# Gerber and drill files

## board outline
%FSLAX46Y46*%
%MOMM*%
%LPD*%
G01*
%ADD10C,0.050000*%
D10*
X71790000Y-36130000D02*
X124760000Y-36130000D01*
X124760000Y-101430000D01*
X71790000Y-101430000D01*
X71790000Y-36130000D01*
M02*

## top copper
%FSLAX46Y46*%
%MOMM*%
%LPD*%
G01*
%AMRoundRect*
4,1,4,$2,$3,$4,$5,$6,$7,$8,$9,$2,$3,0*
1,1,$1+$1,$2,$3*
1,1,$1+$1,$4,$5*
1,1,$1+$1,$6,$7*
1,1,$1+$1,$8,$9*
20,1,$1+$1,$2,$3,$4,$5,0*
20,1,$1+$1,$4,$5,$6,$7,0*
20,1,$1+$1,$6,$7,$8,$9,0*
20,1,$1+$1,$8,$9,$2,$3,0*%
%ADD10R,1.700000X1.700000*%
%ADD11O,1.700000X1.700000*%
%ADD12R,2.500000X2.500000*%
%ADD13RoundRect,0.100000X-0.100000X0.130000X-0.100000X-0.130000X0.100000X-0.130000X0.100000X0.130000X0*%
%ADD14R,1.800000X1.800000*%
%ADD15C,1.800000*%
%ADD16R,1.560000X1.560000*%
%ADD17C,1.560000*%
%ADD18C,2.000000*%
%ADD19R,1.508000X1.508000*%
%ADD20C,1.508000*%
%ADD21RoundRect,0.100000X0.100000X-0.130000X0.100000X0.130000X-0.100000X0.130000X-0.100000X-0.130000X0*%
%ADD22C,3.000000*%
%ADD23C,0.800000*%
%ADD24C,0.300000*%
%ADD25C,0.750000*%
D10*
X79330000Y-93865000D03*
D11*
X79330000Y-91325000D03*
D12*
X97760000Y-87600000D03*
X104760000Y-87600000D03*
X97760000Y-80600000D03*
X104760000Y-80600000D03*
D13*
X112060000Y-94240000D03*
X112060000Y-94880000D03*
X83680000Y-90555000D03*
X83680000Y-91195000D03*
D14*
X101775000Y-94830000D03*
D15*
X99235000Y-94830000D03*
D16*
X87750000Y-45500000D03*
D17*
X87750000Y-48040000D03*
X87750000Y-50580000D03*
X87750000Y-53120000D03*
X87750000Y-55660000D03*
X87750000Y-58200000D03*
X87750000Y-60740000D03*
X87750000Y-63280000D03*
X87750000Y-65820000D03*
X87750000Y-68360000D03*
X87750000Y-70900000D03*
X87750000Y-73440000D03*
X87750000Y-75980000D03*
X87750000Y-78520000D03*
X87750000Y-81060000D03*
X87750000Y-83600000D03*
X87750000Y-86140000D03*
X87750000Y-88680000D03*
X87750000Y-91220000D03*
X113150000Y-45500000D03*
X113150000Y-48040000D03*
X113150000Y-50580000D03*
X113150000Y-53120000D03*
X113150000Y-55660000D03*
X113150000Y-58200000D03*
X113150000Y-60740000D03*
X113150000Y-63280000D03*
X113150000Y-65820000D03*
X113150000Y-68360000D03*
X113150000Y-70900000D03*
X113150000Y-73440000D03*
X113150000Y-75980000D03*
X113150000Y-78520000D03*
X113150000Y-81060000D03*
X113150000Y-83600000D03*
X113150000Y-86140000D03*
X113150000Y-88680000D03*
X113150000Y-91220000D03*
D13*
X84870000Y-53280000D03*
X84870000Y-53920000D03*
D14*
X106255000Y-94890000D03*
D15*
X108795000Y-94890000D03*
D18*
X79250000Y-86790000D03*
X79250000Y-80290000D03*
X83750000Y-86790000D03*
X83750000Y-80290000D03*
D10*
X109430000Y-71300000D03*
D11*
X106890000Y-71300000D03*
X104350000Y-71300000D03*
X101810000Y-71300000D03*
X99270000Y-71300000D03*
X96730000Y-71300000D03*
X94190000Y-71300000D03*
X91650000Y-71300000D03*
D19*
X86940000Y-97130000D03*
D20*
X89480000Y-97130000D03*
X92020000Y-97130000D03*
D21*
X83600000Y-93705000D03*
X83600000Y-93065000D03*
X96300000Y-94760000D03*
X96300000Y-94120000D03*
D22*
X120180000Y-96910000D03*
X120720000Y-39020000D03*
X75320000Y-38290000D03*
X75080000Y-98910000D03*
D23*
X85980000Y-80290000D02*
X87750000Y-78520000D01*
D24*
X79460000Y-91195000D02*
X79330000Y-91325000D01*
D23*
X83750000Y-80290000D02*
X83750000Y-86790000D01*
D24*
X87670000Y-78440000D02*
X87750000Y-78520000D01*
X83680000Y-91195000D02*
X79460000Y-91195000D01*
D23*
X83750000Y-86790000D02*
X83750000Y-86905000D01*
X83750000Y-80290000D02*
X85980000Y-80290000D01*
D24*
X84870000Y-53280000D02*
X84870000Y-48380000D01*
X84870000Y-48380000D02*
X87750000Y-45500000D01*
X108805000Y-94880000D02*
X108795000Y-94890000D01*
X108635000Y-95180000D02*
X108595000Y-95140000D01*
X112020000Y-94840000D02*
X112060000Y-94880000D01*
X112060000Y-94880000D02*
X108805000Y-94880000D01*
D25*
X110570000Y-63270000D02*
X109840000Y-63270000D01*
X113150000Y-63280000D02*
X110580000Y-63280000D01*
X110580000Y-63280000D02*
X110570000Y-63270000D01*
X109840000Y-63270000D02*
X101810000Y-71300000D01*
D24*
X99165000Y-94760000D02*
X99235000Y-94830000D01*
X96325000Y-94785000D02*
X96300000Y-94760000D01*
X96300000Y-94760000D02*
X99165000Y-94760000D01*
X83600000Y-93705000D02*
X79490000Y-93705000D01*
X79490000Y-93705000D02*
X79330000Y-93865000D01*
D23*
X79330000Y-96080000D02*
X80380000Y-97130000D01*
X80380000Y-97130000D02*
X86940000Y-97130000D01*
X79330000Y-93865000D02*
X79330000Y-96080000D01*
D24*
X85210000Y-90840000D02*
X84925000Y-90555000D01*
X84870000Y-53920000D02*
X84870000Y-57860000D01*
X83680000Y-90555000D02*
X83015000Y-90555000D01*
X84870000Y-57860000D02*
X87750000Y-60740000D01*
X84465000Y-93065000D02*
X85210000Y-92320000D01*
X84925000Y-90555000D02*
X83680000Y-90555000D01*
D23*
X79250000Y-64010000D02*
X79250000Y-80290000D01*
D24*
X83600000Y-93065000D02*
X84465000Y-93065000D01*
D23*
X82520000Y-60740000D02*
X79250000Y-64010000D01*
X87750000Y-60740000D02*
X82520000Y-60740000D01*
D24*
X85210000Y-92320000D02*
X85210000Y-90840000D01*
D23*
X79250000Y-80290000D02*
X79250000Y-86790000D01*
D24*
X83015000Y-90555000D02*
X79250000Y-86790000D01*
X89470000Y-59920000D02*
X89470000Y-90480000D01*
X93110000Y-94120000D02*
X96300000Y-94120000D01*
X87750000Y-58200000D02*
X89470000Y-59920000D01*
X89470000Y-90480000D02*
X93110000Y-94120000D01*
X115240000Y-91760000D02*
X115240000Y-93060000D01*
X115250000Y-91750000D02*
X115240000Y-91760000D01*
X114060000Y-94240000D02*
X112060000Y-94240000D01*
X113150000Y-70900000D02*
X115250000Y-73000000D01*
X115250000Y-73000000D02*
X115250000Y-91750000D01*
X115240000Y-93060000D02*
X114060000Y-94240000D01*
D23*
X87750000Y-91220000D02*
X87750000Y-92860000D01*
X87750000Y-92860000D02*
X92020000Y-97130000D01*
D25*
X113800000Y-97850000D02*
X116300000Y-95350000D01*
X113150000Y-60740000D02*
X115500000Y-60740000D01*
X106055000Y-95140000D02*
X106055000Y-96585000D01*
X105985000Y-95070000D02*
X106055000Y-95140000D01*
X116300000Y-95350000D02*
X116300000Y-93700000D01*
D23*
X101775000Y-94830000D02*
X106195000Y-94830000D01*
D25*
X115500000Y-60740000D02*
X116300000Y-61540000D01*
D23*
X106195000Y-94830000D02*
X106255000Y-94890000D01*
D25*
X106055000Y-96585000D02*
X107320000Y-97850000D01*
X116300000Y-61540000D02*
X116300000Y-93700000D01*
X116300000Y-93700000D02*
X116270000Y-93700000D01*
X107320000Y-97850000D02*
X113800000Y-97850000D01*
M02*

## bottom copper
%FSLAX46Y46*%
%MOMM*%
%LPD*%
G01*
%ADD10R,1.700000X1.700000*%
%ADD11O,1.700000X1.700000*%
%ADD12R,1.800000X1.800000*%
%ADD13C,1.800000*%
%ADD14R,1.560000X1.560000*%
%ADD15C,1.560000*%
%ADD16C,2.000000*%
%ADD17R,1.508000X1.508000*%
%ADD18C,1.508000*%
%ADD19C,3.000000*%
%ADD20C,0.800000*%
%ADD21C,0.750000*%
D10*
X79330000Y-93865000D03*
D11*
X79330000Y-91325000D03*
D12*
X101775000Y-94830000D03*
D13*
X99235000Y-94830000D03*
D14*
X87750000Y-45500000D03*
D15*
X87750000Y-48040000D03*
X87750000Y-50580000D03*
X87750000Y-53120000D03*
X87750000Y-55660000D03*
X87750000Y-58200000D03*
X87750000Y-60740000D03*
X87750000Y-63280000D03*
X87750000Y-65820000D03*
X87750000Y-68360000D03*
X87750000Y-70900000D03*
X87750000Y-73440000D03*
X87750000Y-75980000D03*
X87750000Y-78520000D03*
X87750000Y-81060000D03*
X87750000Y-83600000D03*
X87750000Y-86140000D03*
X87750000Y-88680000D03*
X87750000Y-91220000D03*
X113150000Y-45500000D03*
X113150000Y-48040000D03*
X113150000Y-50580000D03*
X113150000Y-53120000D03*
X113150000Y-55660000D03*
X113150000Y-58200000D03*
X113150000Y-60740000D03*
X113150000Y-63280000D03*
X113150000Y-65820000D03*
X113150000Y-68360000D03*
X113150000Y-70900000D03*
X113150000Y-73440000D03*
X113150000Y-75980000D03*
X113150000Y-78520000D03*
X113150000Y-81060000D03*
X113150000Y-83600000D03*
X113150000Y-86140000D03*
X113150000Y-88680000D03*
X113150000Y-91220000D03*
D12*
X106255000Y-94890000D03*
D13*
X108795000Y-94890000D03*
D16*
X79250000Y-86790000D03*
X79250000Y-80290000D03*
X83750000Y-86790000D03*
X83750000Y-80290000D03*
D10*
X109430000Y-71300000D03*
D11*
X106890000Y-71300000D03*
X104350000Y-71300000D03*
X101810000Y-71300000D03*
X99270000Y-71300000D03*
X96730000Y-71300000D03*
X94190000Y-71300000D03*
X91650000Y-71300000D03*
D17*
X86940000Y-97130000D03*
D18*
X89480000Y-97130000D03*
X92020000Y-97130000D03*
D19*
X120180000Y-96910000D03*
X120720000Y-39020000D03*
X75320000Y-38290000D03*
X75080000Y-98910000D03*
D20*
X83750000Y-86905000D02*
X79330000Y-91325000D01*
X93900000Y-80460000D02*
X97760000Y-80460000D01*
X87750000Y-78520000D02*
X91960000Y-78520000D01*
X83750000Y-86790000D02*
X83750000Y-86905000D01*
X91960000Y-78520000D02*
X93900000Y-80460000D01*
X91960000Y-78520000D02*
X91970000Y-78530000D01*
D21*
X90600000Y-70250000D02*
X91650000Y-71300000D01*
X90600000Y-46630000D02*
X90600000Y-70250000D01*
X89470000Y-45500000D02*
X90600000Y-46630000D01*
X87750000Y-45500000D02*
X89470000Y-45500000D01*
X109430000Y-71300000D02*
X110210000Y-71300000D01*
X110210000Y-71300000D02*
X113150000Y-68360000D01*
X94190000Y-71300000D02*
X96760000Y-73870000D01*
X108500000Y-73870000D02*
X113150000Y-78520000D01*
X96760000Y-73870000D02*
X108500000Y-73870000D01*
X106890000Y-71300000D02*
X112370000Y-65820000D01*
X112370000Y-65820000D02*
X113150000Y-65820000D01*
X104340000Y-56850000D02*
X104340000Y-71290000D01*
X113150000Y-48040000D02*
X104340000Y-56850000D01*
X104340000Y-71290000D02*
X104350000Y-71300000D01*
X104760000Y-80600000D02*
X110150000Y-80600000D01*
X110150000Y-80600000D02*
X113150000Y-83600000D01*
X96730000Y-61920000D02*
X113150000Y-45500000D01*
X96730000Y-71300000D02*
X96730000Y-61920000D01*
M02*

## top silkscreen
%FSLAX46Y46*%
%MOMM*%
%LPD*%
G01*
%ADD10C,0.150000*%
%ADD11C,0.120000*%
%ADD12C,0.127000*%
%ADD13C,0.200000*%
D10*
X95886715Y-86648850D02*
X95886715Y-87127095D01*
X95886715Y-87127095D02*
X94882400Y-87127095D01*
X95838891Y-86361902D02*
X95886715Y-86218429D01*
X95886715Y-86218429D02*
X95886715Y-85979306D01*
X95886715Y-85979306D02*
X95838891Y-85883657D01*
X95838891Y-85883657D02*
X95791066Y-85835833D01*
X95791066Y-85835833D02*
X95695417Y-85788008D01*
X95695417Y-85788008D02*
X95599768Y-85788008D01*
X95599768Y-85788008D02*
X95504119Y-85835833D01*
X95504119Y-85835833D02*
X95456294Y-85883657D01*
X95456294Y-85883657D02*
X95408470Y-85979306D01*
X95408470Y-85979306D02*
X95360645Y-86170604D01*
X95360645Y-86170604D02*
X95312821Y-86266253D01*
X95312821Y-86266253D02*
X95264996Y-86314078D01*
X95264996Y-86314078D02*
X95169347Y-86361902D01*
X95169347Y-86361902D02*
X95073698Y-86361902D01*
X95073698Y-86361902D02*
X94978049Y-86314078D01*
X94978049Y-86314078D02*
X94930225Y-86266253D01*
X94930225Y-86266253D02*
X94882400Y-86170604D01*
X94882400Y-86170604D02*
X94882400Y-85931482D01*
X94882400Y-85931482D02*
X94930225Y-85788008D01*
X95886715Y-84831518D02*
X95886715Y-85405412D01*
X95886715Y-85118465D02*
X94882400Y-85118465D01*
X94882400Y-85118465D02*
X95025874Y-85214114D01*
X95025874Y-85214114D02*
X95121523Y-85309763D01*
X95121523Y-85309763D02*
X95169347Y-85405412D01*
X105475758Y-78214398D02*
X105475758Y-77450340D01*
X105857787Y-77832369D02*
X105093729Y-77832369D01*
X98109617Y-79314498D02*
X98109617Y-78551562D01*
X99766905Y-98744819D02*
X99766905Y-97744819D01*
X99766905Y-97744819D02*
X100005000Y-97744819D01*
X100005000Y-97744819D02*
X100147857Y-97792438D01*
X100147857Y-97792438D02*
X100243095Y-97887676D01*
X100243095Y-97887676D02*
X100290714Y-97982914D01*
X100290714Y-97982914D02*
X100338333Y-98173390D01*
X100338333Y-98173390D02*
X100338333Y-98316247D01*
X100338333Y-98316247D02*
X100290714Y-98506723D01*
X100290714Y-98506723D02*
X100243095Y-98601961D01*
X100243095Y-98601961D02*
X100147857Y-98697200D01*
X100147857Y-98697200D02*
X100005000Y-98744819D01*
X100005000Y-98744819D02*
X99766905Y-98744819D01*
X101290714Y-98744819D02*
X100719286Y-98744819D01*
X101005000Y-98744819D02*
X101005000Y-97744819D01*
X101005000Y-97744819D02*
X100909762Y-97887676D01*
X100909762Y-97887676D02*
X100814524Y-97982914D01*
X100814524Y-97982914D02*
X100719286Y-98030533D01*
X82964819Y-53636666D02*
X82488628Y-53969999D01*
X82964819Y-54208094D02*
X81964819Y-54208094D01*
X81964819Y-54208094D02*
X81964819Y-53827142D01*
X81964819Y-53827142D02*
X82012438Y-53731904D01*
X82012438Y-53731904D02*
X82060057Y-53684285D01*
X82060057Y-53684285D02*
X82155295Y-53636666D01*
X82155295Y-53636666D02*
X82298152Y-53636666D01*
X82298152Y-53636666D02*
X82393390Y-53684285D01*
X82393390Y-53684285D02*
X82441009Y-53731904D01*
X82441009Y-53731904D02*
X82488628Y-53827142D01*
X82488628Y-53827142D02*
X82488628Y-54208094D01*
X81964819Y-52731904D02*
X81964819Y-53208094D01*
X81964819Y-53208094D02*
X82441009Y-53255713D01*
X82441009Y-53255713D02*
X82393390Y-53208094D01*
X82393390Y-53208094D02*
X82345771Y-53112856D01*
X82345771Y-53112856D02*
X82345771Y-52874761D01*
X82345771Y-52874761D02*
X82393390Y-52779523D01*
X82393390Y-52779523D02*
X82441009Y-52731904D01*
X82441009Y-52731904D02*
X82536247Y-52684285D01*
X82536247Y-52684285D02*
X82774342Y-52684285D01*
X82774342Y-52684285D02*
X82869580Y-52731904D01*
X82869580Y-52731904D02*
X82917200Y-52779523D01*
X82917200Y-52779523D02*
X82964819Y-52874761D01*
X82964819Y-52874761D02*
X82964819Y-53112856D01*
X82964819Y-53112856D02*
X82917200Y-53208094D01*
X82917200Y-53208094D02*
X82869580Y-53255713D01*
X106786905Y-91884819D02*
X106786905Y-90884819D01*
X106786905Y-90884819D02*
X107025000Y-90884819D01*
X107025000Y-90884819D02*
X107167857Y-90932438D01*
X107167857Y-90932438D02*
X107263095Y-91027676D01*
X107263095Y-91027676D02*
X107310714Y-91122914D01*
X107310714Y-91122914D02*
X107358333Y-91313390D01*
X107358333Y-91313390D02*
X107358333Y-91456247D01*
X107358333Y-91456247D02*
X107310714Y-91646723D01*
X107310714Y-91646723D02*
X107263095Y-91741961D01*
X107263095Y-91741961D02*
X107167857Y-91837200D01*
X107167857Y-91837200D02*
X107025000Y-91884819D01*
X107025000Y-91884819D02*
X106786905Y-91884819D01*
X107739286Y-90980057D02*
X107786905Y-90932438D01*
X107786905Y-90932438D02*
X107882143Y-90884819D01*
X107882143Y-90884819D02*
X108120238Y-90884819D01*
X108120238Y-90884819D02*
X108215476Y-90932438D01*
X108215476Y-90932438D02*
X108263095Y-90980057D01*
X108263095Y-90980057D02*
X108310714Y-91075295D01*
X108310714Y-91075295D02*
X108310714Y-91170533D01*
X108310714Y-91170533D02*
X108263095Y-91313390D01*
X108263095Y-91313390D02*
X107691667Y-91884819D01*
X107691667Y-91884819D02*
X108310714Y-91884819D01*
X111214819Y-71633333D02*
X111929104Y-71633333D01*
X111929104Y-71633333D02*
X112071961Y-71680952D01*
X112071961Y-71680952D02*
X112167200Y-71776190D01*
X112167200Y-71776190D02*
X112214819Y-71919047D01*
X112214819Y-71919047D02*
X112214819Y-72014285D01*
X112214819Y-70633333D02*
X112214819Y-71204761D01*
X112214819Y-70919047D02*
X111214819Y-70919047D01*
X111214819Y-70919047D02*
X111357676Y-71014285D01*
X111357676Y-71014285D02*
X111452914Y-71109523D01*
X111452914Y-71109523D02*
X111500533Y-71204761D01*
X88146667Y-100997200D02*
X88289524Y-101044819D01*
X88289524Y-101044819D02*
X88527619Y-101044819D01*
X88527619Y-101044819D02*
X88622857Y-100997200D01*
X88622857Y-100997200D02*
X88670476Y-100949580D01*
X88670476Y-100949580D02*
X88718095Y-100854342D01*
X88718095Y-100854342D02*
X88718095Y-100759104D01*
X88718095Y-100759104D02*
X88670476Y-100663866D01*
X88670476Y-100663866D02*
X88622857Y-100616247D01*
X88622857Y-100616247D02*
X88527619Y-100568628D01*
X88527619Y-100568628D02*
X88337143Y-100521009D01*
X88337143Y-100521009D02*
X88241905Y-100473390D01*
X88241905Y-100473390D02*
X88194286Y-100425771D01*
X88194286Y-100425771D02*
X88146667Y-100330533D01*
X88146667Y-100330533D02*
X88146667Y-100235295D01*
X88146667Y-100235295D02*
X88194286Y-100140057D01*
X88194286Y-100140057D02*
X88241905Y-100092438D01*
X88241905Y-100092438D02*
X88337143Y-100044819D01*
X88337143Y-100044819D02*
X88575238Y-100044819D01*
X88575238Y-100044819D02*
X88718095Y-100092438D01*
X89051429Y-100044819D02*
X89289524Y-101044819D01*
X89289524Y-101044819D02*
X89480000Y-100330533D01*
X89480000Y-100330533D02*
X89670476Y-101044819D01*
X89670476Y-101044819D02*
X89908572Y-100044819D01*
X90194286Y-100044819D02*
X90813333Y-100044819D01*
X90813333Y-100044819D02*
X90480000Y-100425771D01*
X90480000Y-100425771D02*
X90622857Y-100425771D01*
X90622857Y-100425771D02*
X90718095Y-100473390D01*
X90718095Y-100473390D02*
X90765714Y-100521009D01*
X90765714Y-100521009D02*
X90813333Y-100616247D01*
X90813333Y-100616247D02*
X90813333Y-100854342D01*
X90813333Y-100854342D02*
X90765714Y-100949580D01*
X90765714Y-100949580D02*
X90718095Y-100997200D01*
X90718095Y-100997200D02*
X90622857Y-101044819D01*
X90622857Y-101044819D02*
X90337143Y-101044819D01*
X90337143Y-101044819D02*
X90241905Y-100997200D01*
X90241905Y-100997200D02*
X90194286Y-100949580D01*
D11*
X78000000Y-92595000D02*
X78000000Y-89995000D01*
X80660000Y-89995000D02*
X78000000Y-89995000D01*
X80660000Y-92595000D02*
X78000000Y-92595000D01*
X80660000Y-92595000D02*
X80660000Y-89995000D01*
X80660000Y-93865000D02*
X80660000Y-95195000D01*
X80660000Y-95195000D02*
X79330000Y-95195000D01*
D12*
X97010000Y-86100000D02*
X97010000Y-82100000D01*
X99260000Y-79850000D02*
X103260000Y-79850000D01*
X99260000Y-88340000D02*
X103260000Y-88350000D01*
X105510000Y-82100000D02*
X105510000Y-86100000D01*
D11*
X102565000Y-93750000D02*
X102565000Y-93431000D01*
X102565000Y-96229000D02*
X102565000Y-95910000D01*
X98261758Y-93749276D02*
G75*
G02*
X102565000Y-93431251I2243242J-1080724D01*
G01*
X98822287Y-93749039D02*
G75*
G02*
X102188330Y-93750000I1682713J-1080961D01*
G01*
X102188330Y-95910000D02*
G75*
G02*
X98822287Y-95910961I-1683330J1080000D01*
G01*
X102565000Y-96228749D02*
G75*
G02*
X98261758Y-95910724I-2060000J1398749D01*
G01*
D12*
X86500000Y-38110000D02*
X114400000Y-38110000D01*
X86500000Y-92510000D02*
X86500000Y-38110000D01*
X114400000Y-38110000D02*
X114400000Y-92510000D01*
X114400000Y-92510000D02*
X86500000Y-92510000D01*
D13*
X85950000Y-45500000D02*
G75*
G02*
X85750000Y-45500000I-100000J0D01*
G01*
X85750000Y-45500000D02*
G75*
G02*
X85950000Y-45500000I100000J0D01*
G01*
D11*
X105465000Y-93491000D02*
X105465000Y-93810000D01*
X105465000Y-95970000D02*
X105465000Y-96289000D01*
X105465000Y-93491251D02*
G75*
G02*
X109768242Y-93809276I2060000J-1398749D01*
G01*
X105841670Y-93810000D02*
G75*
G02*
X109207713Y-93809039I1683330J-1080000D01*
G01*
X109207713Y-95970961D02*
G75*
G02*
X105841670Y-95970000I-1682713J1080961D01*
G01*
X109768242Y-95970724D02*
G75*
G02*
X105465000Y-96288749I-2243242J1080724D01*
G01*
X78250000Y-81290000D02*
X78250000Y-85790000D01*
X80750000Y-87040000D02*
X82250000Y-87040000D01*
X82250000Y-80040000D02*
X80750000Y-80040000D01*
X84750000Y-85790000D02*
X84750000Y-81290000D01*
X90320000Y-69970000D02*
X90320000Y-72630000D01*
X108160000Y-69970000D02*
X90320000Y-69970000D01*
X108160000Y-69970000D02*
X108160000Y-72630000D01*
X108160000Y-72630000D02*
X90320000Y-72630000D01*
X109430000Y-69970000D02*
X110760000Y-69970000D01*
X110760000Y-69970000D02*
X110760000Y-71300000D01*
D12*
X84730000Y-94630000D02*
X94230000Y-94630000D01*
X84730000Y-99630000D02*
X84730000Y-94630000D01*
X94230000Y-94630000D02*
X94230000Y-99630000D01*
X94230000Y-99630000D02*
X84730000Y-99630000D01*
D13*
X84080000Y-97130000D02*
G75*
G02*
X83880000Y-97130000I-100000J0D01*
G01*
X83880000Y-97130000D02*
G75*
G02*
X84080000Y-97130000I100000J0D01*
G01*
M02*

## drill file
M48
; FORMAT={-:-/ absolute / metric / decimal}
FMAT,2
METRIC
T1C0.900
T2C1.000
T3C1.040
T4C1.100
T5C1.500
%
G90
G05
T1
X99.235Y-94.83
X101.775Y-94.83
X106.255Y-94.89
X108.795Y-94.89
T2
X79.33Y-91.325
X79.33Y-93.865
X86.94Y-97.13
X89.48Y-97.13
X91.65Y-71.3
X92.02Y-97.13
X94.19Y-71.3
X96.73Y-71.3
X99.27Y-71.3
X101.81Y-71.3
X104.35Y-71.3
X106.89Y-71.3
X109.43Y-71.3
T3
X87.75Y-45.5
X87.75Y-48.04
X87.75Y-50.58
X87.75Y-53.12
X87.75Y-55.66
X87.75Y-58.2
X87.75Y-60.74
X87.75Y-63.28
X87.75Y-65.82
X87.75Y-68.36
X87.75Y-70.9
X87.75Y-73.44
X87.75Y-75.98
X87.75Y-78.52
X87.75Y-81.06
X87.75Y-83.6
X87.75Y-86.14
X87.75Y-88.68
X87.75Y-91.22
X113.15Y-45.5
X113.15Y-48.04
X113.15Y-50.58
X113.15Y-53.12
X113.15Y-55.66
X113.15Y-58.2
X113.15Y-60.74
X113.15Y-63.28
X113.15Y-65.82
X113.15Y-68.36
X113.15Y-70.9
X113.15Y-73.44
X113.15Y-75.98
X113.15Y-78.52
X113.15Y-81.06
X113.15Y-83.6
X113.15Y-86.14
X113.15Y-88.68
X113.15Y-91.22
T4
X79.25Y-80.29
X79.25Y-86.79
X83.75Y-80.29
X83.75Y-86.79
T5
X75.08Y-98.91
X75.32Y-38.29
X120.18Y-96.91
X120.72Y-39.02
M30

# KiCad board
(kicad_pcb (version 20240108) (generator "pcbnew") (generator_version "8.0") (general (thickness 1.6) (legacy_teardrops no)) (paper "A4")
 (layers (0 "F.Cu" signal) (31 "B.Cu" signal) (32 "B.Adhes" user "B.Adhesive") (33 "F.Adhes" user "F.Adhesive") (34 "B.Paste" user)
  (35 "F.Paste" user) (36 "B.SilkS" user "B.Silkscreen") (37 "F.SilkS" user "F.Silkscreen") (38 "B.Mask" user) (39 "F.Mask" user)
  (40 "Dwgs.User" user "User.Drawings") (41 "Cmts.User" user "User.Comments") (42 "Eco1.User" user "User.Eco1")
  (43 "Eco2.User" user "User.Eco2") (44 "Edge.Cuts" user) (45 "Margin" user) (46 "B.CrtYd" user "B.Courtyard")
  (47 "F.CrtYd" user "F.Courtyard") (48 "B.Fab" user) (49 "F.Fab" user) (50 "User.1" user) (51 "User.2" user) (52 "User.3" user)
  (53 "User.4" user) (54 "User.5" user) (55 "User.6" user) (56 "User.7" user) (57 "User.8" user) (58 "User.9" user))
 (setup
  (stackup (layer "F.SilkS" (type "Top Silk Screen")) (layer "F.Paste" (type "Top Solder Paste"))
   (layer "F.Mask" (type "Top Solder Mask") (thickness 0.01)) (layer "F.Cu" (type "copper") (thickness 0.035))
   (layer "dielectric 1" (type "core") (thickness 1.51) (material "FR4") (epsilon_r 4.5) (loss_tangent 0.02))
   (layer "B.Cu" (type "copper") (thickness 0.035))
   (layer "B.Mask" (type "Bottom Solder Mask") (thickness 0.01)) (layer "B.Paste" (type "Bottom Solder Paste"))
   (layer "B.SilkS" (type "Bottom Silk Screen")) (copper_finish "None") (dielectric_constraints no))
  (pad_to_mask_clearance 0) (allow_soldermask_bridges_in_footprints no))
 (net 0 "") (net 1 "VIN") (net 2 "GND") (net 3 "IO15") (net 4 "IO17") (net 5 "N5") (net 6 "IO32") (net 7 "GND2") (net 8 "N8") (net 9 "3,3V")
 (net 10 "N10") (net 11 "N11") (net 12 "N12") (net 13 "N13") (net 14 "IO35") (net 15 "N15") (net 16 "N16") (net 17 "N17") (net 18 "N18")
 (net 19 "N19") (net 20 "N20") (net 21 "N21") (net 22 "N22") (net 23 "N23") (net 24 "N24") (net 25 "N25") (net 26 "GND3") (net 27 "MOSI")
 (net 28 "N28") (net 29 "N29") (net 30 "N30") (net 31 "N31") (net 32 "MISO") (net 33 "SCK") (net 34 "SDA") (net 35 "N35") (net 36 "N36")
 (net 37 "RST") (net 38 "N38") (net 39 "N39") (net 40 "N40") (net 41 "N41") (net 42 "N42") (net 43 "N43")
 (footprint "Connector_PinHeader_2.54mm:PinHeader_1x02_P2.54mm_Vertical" (layer "F.Cu") (at 79.33 93.865 180)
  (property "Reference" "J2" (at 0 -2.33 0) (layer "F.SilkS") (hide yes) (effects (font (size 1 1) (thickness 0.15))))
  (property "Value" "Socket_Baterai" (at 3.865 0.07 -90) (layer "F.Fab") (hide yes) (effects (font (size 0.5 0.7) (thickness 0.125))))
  (fp_line (start 1.33 1.27) (end 1.33 3.87) (stroke (width 0.12) (type solid)) (layer "F.SilkS"))
  (fp_line (start -1.33 3.87) (end 1.33 3.87) (stroke (width 0.12) (type solid)) (layer "F.SilkS"))
  (fp_line (start -1.33 1.27) (end 1.33 1.27) (stroke (width 0.12) (type solid)) (layer "F.SilkS"))
  (fp_line (start -1.33 1.27) (end -1.33 3.87) (stroke (width 0.12) (type solid)) (layer "F.SilkS"))
  (fp_line (start -1.33 0) (end -1.33 -1.33) (stroke (width 0.12) (type solid)) (layer "F.SilkS"))
  (fp_line (start -1.33 -1.33) (end 0 -1.33) (stroke (width 0.12) (type solid)) (layer "F.SilkS"))
  (pad "1" thru_hole rect (at 0 0 180) (size 1.7 1.7) (drill 1) (layers "*.Cu" "*.Mask") (remove_unused_layers no) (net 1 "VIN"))
  (pad "2" thru_hole oval (at 0 2.54 180) (size 1.7 1.7) (drill 1) (layers "*.Cu" "*.Mask") (remove_unused_layers no) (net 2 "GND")))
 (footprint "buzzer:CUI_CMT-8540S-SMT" (layer "F.Cu") (at 101.26 84.1 90)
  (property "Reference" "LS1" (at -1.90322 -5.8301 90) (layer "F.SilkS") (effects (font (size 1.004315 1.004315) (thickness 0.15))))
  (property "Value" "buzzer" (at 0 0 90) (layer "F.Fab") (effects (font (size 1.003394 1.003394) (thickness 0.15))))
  (fp_line (start -2 -4.25) (end 2 -4.25) (stroke (width 0.127) (type solid)) (layer "F.SilkS"))
  (fp_line (start 4.25 -2) (end 4.25 2) (stroke (width 0.127) (type solid)) (layer "F.SilkS"))
  (fp_line (start -4.24 -2) (end -4.25 2) (stroke (width 0.127) (type solid)) (layer "F.SilkS"))
  (fp_line (start 2 4.25) (end -2 4.25) (stroke (width 0.127) (type solid)) (layer "F.SilkS"))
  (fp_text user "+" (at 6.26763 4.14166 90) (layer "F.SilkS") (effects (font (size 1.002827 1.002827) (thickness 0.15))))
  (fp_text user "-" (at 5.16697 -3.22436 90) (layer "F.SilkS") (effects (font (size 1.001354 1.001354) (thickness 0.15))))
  (pad "1" smd rect (at -3.5 -3.5 90) (size 2.5 2.5) (layers "F.Cu" "F.Paste" "F.Mask") (solder_mask_margin 0.102))
  (pad "2" smd rect (at -3.5 3.5 90) (size 2.5 2.5) (layers "F.Cu" "F.Paste" "F.Mask") (solder_mask_margin 0.102))
  (pad "N" smd rect (at 3.5 -3.5 90) (size 2.5 2.5) (layers "F.Cu" "F.Paste" "F.Mask") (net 2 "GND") (solder_mask_margin 0.102))
  (pad "P" smd rect (at 3.5 3.5 90) (size 2.5 2.5) (layers "F.Cu" "F.Paste" "F.Mask") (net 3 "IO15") (solder_mask_margin 0.102)))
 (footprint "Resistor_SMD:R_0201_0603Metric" (layer "F.Cu") (at 112.06 94.56 -90)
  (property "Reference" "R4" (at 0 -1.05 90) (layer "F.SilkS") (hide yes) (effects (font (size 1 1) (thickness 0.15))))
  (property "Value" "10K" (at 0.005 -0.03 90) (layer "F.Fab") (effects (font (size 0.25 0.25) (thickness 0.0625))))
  (pad "" smd roundrect (at -0.345 0 270) (size 0.318 0.36) (layers "F.Paste") (roundrect_rratio 0.25))
  (pad "" smd roundrect (at 0.345 0 270) (size 0.318 0.36) (layers "F.Paste") (roundrect_rratio 0.25))
  (pad "1" smd roundrect (at -0.32 0 270) (size 0.46 0.4) (layers "F.Cu" "F.Mask") (roundrect_rratio 0.25) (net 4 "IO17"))
  (pad "2" smd roundrect (at 0.32 0 270) (size 0.46 0.4) (layers "F.Cu" "F.Mask") (roundrect_rratio 0.25) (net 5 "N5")))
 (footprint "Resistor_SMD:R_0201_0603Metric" (layer "F.Cu") (at 83.68 90.875 -90)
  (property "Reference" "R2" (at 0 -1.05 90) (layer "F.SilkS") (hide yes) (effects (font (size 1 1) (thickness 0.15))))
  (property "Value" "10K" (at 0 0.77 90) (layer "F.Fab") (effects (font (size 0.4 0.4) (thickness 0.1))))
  (pad "" smd roundrect (at -0.345 0 270) (size 0.318 0.36) (layers "F.Paste") (roundrect_rratio 0.25))
  (pad "" smd roundrect (at 0.345 0 270) (size 0.318 0.36) (layers "F.Paste") (roundrect_rratio 0.25))
  (pad "1" smd roundrect (at -0.32 0 270) (size 0.46 0.4) (layers "F.Cu" "F.Mask") (roundrect_rratio 0.25) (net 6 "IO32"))
  (pad "2" smd roundrect (at 0.32 0 270) (size 0.46 0.4) (layers "F.Cu" "F.Mask") (roundrect_rratio 0.25) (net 2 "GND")))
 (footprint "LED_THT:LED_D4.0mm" (layer "F.Cu") (at 101.775 94.83 180)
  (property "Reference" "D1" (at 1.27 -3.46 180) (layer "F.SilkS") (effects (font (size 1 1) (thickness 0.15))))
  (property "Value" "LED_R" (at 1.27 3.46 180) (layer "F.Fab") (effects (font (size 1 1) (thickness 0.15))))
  (fp_line (start -0.79 1.08) (end -0.79 1.399) (stroke (width 0.12) (type solid)) (layer "F.SilkS"))
  (fp_line (start -0.79 -1.399) (end -0.79 -1.08) (stroke (width 0.12) (type solid)) (layer "F.SilkS"))
  (fp_arc (start 3.513242 1.080724) (mid 1.453519 2.483228) (end -0.79 1.398749) (stroke (width 0.12) (type solid)) (layer "F.SilkS"))
  (fp_arc (start 2.952713 1.080961) (mid 1.269429 2) (end -0.41333 1.08) (stroke (width 0.12) (type solid)) (layer "F.SilkS"))
  (fp_arc (start -0.41333 -1.08) (mid 1.269429 -2) (end 2.952713 -1.080961) (stroke (width 0.12) (type solid)) (layer "F.SilkS"))
  (fp_arc (start -0.79 -1.398749) (mid 1.453519 -2.483228) (end 3.513242 -1.080724) (stroke (width 0.12) (type solid)) (layer "F.SilkS"))
  (pad "1" thru_hole rect (at 0 0 180) (size 1.8 1.8) (drill 0.9) (layers "*.Cu" "*.Mask") (remove_unused_layers no) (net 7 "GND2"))
  (pad "2" thru_hole circle (at 2.54 0 180) (size 1.8 1.8) (drill 0.9) (layers "*.Cu" "*.Mask") (remove_unused_layers no) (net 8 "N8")))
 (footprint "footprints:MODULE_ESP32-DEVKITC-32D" (layer "F.Cu") (at 100.45 65.26)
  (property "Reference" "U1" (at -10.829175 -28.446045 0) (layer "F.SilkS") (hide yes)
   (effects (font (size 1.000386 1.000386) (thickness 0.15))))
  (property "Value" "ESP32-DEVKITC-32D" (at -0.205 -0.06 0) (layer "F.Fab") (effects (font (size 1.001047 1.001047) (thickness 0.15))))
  (fp_line (start -13.95 -27.15) (end 13.95 -27.15) (stroke (width 0.127) (type solid)) (layer "F.SilkS"))
  (fp_line (start -13.95 27.25) (end -13.95 -27.15) (stroke (width 0.127) (type solid)) (layer "F.SilkS"))
  (fp_line (start 13.95 -27.15) (end 13.95 27.25) (stroke (width 0.127) (type solid)) (layer "F.SilkS"))
  (fp_line (start 13.95 27.25) (end -13.95 27.25) (stroke (width 0.127) (type solid)) (layer "F.SilkS"))
  (fp_circle (center -14.6 -19.76) (end -14.5 -19.76) (stroke (width 0.2) (type solid)) (fill none) (layer "F.SilkS"))
  (pad "J2-1" thru_hole rect (at -12.7 -19.76) (size 1.56 1.56) (drill 1.04) (layers "*.Cu" "*.Mask") (remove_unused_layers no)
   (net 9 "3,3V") (solder_mask_margin 0.102))
  (pad "J2-2" thru_hole circle (at -12.7 -17.22) (size 1.56 1.56) (drill 1.04) (layers "*.Cu" "*.Mask") (remove_unused_layers no)
   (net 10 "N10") (solder_mask_margin 0.102))
  (pad "J2-3" thru_hole circle (at -12.7 -14.68) (size 1.56 1.56) (drill 1.04) (layers "*.Cu" "*.Mask") (remove_unused_layers no)
   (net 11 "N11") (solder_mask_margin 0.102))
  (pad "J2-4" thru_hole circle (at -12.7 -12.14) (size 1.56 1.56) (drill 1.04) (layers "*.Cu" "*.Mask") (remove_unused_layers no)
   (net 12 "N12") (solder_mask_margin 0.102))
  (pad "J2-5" thru_hole circle (at -12.7 -9.6) (size 1.56 1.56) (drill 1.04) (layers "*.Cu" "*.Mask") (remove_unused_layers no)
   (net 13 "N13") (solder_mask_margin 0.102))
  (pad "J2-6" thru_hole circle (at -12.7 -7.06) (size 1.56 1.56) (drill 1.04) (layers "*.Cu" "*.Mask") (remove_unused_layers no)
   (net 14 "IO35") (solder_mask_margin 0.102))
  (pad "J2-7" thru_hole circle (at -12.7 -4.52) (size 1.56 1.56) (drill 1.04) (layers "*.Cu" "*.Mask") (remove_unused_layers no)
   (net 6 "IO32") (solder_mask_margin 0.102))
  (pad "J2-8" thru_hole circle (at -12.7 -1.98) (size 1.56 1.56) (drill 1.04) (layers "*.Cu" "*.Mask") (remove_unused_layers no)
   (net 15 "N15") (solder_mask_margin 0.102))
  (pad "J2-9" thru_hole circle (at -12.7 0.56) (size 1.56 1.56) (drill 1.04) (layers "*.Cu" "*.Mask") (remove_unused_layers no)
   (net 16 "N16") (solder_mask_margin 0.102))
  (pad "J2-10" thru_hole circle (at -12.7 3.1) (size 1.56 1.56) (drill 1.04) (layers "*.Cu" "*.Mask") (remove_unused_layers no)
   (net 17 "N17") (solder_mask_margin 0.102))
  (pad "J2-11" thru_hole circle (at -12.7 5.64) (size 1.56 1.56) (drill 1.04) (layers "*.Cu" "*.Mask") (remove_unused_layers no)
   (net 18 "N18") (solder_mask_margin 0.102))
  (pad "J2-12" thru_hole circle (at -12.7 8.18) (size 1.56 1.56) (drill 1.04) (layers "*.Cu" "*.Mask") (remove_unused_layers no)
   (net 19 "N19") (solder_mask_margin 0.102))
  (pad "J2-13" thru_hole circle (at -12.7 10.72) (size 1.56 1.56) (drill 1.04) (layers "*.Cu" "*.Mask") (remove_unused_layers no)
   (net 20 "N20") (solder_mask_margin 0.102))
  (pad "J2-14" thru_hole circle (at -12.7 13.26) (size 1.56 1.56) (drill 1.04) (layers "*.Cu" "*.Mask") (remove_unused_layers no)
   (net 2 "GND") (solder_mask_margin 0.102))
  (pad "J2-15" thru_hole circle (at -12.7 15.8) (size 1.56 1.56) (drill 1.04) (layers "*.Cu" "*.Mask") (remove_unused_layers no)
   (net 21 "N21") (solder_mask_margin 0.102))
  (pad "J2-16" thru_hole circle (at -12.7 18.34) (size 1.56 1.56) (drill 1.04) (layers "*.Cu" "*.Mask") (remove_unused_layers no)
   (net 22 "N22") (solder_mask_margin 0.102))
  (pad "J2-17" thru_hole circle (at -12.7 20.88) (size 1.56 1.56) (drill 1.04) (layers "*.Cu" "*.Mask") (remove_unused_layers no)
   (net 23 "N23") (solder_mask_margin 0.102))
  (pad "J2-18" thru_hole circle (at -12.7 23.42) (size 1.56 1.56) (drill 1.04) (layers "*.Cu" "*.Mask") (remove_unused_layers no)
   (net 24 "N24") (solder_mask_margin 0.102))
  (pad "J2-19" thru_hole circle (at -12.7 25.96) (size 1.56 1.56) (drill 1.04) (layers "*.Cu" "*.Mask") (remove_unused_layers no)
   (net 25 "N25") (solder_mask_margin 0.102))
  (pad "J3-1" thru_hole circle (at 12.7 -19.76) (size 1.56 1.56) (drill 1.04) (layers "*.Cu" "*.Mask") (remove_unused_layers no)
   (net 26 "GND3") (solder_mask_margin 0.102))
  (pad "J3-2" thru_hole circle (at 12.7 -17.22) (size 1.56 1.56) (drill 1.04) (layers "*.Cu" "*.Mask") (remove_unused_layers no)
   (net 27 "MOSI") (solder_mask_margin 0.102))
  (pad "J3-3" thru_hole circle (at 12.7 -14.68) (size 1.56 1.56) (drill 1.04) (layers "*.Cu" "*.Mask") (remove_unused_layers no)
   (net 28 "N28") (solder_mask_margin 0.102))
  (pad "J3-4" thru_hole circle (at 12.7 -12.14) (size 1.56 1.56) (drill 1.04) (layers "*.Cu" "*.Mask") (remove_unused_layers no)
   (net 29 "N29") (solder_mask_margin 0.102))
  (pad "J3-5" thru_hole circle (at 12.7 -9.6) (size 1.56 1.56) (drill 1.04) (layers "*.Cu" "*.Mask") (remove_unused_layers no)
   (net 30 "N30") (solder_mask_margin 0.102))
  (pad "J3-6" thru_hole circle (at 12.7 -7.06) (size 1.56 1.56) (drill 1.04) (layers "*.Cu" "*.Mask") (remove_unused_layers no)
   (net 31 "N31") (solder_mask_margin 0.102))
  (pad "J3-7" thru_hole circle (at 12.7 -4.52) (size 1.56 1.56) (drill 1.04) (layers "*.Cu" "*.Mask") (remove_unused_layers no)
   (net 7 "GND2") (solder_mask_margin 0.102))
  (pad "J3-8" thru_hole circle (at 12.7 -1.98) (size 1.56 1.56) (drill 1.04) (layers "*.Cu" "*.Mask") (remove_unused_layers no)
   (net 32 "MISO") (solder_mask_margin 0.102))
  (pad "J3-9" thru_hole circle (at 12.7 0.56) (size 1.56 1.56) (drill 1.04) (layers "*.Cu" "*.Mask") (remove_unused_layers no)
   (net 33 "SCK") (solder_mask_margin 0.102))
  (pad "J3-10" thru_hole circle (at 12.7 3.1) (size 1.56 1.56) (drill 1.04) (layers "*.Cu" "*.Mask") (remove_unused_layers no)
   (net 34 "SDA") (solder_mask_margin 0.102))
  (pad "J3-11" thru_hole circle (at 12.7 5.64) (size 1.56 1.56) (drill 1.04) (layers "*.Cu" "*.Mask") (remove_unused_layers no)
   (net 4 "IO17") (solder_mask_margin 0.102))
  (pad "J3-12" thru_hole circle (at 12.7 8.18) (size 1.56 1.56) (drill 1.04) (layers "*.Cu" "*.Mask") (remove_unused_layers no)
   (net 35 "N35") (solder_mask_margin 0.102))
  (pad "J3-13" thru_hole circle (at 12.7 10.72) (size 1.56 1.56) (drill 1.04) (layers "*.Cu" "*.Mask") (remove_unused_layers no)
   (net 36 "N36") (solder_mask_margin 0.102))
  (pad "J3-14" thru_hole circle (at 12.7 13.26) (size 1.56 1.56) (drill 1.04) (layers "*.Cu" "*.Mask") (remove_unused_layers no)
   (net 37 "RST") (solder_mask_margin 0.102))
  (pad "J3-15" thru_hole circle (at 12.7 15.8) (size 1.56 1.56) (drill 1.04) (layers "*.Cu" "*.Mask") (remove_unused_layers no)
   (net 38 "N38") (solder_mask_margin 0.102))
  (pad "J3-16" thru_hole circle (at 12.7 18.34) (size 1.56 1.56) (drill 1.04) (layers "*.Cu" "*.Mask") (remove_unused_layers no)
   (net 3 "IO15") (solder_mask_margin 0.102))
  (pad "J3-17" thru_hole circle (at 12.7 20.88) (size 1.56 1.56) (drill 1.04) (layers "*.Cu" "*.Mask") (remove_unused_layers no)
   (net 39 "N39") (solder_mask_margin 0.102))
  (pad "J3-18" thru_hole circle (at 12.7 23.42) (size 1.56 1.56) (drill 1.04) (layers "*.Cu" "*.Mask") (remove_unused_layers no)
   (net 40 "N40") (solder_mask_margin 0.102))
  (pad "J3-19" thru_hole circle (at 12.7 25.96) (size 1.56 1.56) (drill 1.04) (layers "*.Cu" "*.Mask") (remove_unused_layers no)
   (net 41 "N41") (solder_mask_margin 0.102)))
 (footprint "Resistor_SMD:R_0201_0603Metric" (layer "F.Cu") (at 84.87 53.6 -90)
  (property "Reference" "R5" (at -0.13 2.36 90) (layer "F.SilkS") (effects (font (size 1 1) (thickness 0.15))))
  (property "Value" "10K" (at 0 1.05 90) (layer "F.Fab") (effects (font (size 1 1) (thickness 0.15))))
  (pad "" smd roundrect (at -0.345 0 270) (size 0.318 0.36) (layers "F.Paste") (roundrect_rratio 0.25))
  (pad "" smd roundrect (at 0.345 0 270) (size 0.318 0.36) (layers "F.Paste") (roundrect_rratio 0.25))
  (pad "1" smd roundrect (at -0.32 0 270) (size 0.46 0.4) (layers "F.Cu" "F.Mask") (roundrect_rratio 0.25) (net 9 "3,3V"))
  (pad "2" smd roundrect (at 0.32 0 270) (size 0.46 0.4) (layers "F.Cu" "F.Mask") (roundrect_rratio 0.25) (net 6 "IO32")))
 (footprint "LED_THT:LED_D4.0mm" (layer "F.Cu") (at 106.255 94.89)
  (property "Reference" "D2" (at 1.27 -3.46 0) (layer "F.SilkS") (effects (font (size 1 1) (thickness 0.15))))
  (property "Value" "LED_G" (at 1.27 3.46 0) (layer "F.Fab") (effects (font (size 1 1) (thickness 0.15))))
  (fp_line (start -0.79 -1.399) (end -0.79 -1.08) (stroke (width 0.12) (type solid)) (layer "F.SilkS"))
  (fp_line (start -0.79 1.08) (end -0.79 1.399) (stroke (width 0.12) (type solid)) (layer "F.SilkS"))
  (fp_arc (start -0.79 -1.398749) (mid 1.453519 -2.483228) (end 3.513242 -1.080724) (stroke (width 0.12) (type solid)) (layer "F.SilkS"))
  (fp_arc (start -0.41333 -1.08) (mid 1.269429 -2) (end 2.952713 -1.080961) (stroke (width 0.12) (type solid)) (layer "F.SilkS"))
  (fp_arc (start 2.952713 1.080961) (mid 1.269429 2) (end -0.41333 1.08) (stroke (width 0.12) (type solid)) (layer "F.SilkS"))
  (fp_arc (start 3.513242 1.080724) (mid 1.453519 2.483228) (end -0.79 1.398749) (stroke (width 0.12) (type solid)) (layer "F.SilkS"))
  (pad "1" thru_hole rect (at 0 0) (size 1.8 1.8) (drill 0.9) (layers "*.Cu" "*.Mask") (remove_unused_layers no) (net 7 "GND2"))
  (pad "2" thru_hole circle (at 2.54 0) (size 1.8 1.8) (drill 0.9) (layers "*.Cu" "*.Mask") (remove_unused_layers no) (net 5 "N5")))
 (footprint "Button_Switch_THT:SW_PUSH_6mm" (layer "F.Cu") (at 79.25 86.79 90)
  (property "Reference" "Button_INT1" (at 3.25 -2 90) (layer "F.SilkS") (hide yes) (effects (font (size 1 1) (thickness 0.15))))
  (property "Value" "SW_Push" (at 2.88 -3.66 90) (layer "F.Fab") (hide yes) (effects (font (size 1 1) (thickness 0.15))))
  (fp_line (start 5.5 -1) (end 1 -1) (stroke (width 0.12) (type solid)) (layer "F.SilkS"))
  (fp_line (start -0.25 1.5) (end -0.25 3) (stroke (width 0.12) (type solid)) (layer "F.SilkS"))
  (fp_line (start 6.75 3) (end 6.75 1.5) (stroke (width 0.12) (type solid)) (layer "F.SilkS"))
  (fp_line (start 1 5.5) (end 5.5 5.5) (stroke (width 0.12) (type solid)) (layer "F.SilkS"))
  (pad "1" thru_hole circle (at 0 0 180) (size 2 2) (drill 1.1) (layers "*.Cu" "*.Mask") (remove_unused_layers no) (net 6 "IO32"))
  (pad "1" thru_hole circle (at 6.5 0 180) (size 2 2) (drill 1.1) (layers "*.Cu" "*.Mask") (remove_unused_layers no) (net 6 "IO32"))
  (pad "2" thru_hole circle (at 0 4.5 180) (size 2 2) (drill 1.1) (layers "*.Cu" "*.Mask") (remove_unused_layers no) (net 2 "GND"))
  (pad "2" thru_hole circle (at 6.5 4.5 180) (size 2 2) (drill 1.1) (layers "*.Cu" "*.Mask") (remove_unused_layers no) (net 2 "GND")))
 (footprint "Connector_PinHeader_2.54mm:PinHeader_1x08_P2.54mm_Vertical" (layer "F.Cu") (at 109.43 71.3 -90)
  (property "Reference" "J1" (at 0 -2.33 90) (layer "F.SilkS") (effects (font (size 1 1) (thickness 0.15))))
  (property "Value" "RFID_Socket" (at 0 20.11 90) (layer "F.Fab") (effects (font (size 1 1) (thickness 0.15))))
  (fp_line (start -1.33 19.11) (end 1.33 19.11) (stroke (width 0.12) (type solid)) (layer "F.SilkS"))
  (fp_line (start -1.33 1.27) (end -1.33 19.11) (stroke (width 0.12) (type solid)) (layer "F.SilkS"))
  (fp_line (start -1.33 1.27) (end 1.33 1.27) (stroke (width 0.12) (type solid)) (layer "F.SilkS"))
  (fp_line (start 1.33 1.27) (end 1.33 19.11) (stroke (width 0.12) (type solid)) (layer "F.SilkS"))
  (fp_line (start -1.33 0) (end -1.33 -1.33) (stroke (width 0.12) (type solid)) (layer "F.SilkS"))
  (fp_line (start -1.33 -1.33) (end 0 -1.33) (stroke (width 0.12) (type solid)) (layer "F.SilkS"))
  (pad "1" thru_hole rect (at 0 0 270) (size 1.7 1.7) (drill 1) (layers "*.Cu" "*.Mask") (remove_unused_layers no) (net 34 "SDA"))
  (pad "2" thru_hole oval (at 0 2.54 270) (size 1.7 1.7) (drill 1) (layers "*.Cu" "*.Mask") (remove_unused_layers no) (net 33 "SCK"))
  (pad "3" thru_hole oval (at 0 5.08 270) (size 1.7 1.7) (drill 1) (layers "*.Cu" "*.Mask") (remove_unused_layers no) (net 27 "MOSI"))
  (pad "4" thru_hole oval (at 0 7.62 270) (size 1.7 1.7) (drill 1) (layers "*.Cu" "*.Mask") (remove_unused_layers no) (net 32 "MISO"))
  (pad "5" thru_hole oval (at 0 10.16 270) (size 1.7 1.7) (drill 1) (layers "*.Cu" "*.Mask") (remove_unused_layers no) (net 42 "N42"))
  (pad "6" thru_hole oval (at 0 12.7 270) (size 1.7 1.7) (drill 1) (layers "*.Cu" "*.Mask") (remove_unused_layers no) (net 26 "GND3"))
  (pad "7" thru_hole oval (at 0 15.24 270) (size 1.7 1.7) (drill 1) (layers "*.Cu" "*.Mask") (remove_unused_layers no) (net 37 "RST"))
  (pad "8" thru_hole oval (at 0 17.78 270) (size 1.7 1.7) (drill 1) (layers "*.Cu" "*.Mask") (remove_unused_layers no) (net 9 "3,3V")))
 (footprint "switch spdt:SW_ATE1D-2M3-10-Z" (layer "F.Cu") (at 89.48 97.13 180)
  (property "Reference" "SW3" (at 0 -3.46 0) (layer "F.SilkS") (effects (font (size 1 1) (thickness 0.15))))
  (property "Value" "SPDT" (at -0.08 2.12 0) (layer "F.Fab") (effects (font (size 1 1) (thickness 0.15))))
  (fp_line (start 4.75 2.5) (end -4.75 2.5) (stroke (width 0.127) (type solid)) (layer "F.SilkS"))
  (fp_line (start 4.75 -2.5) (end 4.75 2.5) (stroke (width 0.127) (type solid)) (layer "F.SilkS"))
  (fp_line (start -4.75 2.5) (end -4.75 -2.5) (stroke (width 0.127) (type solid)) (layer "F.SilkS"))
  (fp_line (start -4.75 -2.5) (end 4.75 -2.5) (stroke (width 0.127) (type solid)) (layer "F.SilkS"))
  (fp_circle (center 5.5 0) (end 5.6 0) (stroke (width 0.2) (type solid)) (fill none) (layer "F.SilkS"))
  (pad "1" thru_hole rect (at 2.54 0 180) (size 1.508 1.508) (drill 1) (layers "*.Cu" "*.Mask") (remove_unused_layers no) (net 1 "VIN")
   (solder_mask_margin 0.102))
  (pad "2" thru_hole circle (at 0 0 180) (size 1.508 1.508) (drill 1) (layers "*.Cu" "*.Mask") (remove_unused_layers no) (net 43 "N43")
   (solder_mask_margin 0.102))
  (pad "3" thru_hole circle (at -2.54 0 180) (size 1.508 1.508) (drill 1) (layers "*.Cu" "*.Mask") (remove_unused_layers no) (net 25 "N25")
   (solder_mask_margin 0.102)))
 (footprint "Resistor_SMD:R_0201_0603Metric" (layer "F.Cu") (at 83.6 93.385 90)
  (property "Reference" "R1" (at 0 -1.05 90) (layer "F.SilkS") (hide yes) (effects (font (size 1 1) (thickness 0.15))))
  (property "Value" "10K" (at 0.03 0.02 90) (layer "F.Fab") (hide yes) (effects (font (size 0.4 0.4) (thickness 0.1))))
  (pad "" smd roundrect (at -0.345 0 90) (size 0.318 0.36) (layers "F.Paste") (roundrect_rratio 0.25))
  (pad "" smd roundrect (at 0.345 0 90) (size 0.318 0.36) (layers "F.Paste") (roundrect_rratio 0.25))
  (pad "1" smd roundrect (at -0.32 0 90) (size 0.46 0.4) (layers "F.Cu" "F.Mask") (roundrect_rratio 0.25) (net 1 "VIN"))
  (pad "2" smd roundrect (at 0.32 0 90) (size 0.46 0.4) (layers "F.Cu" "F.Mask") (roundrect_rratio 0.25) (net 6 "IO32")))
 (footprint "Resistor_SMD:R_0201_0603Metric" (layer "F.Cu") (at 96.3 94.44 90)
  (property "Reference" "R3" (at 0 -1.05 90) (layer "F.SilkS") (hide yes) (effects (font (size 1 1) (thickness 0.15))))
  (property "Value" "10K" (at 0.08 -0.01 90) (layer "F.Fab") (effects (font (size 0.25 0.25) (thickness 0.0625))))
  (pad "" smd roundrect (at -0.345 0 90) (size 0.318 0.36) (layers "F.Paste") (roundrect_rratio 0.25))
  (pad "" smd roundrect (at 0.345 0 90) (size 0.318 0.36) (layers "F.Paste") (roundrect_rratio 0.25))
  (pad "1" smd roundrect (at -0.32 0 90) (size 0.46 0.4) (layers "F.Cu" "F.Mask") (roundrect_rratio 0.25) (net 8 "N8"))
  (pad "2" smd roundrect (at 0.32 0 90) (size 0.46 0.4) (layers "F.Cu" "F.Mask") (roundrect_rratio 0.25) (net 14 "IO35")))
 (gr_rect (start 71.79 36.13) (end 124.76 101.43) (stroke (width 0.05) (type default)) (fill none) (layer "Edge.Cuts"))
 (via (at 120.18 96.91) (size 3) (drill 1.5) (layers "F.Cu" "B.Cu") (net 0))
 (via (at 120.72 39.02) (size 3) (drill 1.5) (layers "F.Cu" "B.Cu") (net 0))
 (via (at 75.32 38.29) (size 3) (drill 1.5) (layers "F.Cu" "B.Cu") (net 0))
 (via (at 75.08 98.91) (size 3) (drill 1.5) (layers "F.Cu" "B.Cu") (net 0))
 (segment (start 85.98 80.29) (end 87.75 78.52) (width 0.8) (layer "F.Cu") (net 2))
 (segment (start 79.46 91.195) (end 79.33 91.325) (width 0.3) (layer "F.Cu") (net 2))
 (segment (start 83.75 80.29) (end 83.75 86.79) (width 0.8) (layer "F.Cu") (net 2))
 (segment (start 87.67 78.44) (end 87.75 78.52) (width 0.3) (layer "F.Cu") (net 2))
 (segment (start 83.68 91.195) (end 79.46 91.195) (width 0.3) (layer "F.Cu") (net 2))
 (segment (start 83.75 86.79) (end 83.75 86.905) (width 0.8) (layer "F.Cu") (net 2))
 (segment (start 83.75 80.29) (end 85.98 80.29) (width 0.8) (layer "F.Cu") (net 2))
 (segment (start 83.75 86.905) (end 79.33 91.325) (width 0.8) (layer "B.Cu") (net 2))
 (segment (start 93.9 80.46) (end 97.76 80.46) (width 0.8) (layer "B.Cu") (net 2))
 (segment (start 87.75 78.52) (end 91.96 78.52) (width 0.8) (layer "B.Cu") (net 2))
 (segment (start 83.75 86.79) (end 83.75 86.905) (width 0.8) (layer "B.Cu") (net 2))
 (segment (start 91.96 78.52) (end 93.9 80.46) (width 0.8) (layer "B.Cu") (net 2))
 (segment (start 91.96 78.52) (end 91.97 78.53) (width 0.8) (layer "B.Cu") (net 2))
 (segment (start 84.87 53.28) (end 84.87 48.38) (width 0.3) (layer "F.Cu") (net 9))
 (segment (start 84.87 48.38) (end 87.75 45.5) (width 0.3) (layer "F.Cu") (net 9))
 (segment (start 90.6 70.25) (end 91.65 71.3) (width 0.75) (layer "B.Cu") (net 9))
 (segment (start 90.6 46.63) (end 90.6 70.25) (width 0.75) (layer "B.Cu") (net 9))
 (segment (start 89.47 45.5) (end 90.6 46.63) (width 0.75) (layer "B.Cu") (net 9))
 (segment (start 87.75 45.5) (end 89.47 45.5) (width 0.75) (layer "B.Cu") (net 9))
 (segment (start 108.805 94.88) (end 108.795 94.89) (width 0.3) (layer "F.Cu") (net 5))
 (segment (start 108.635 95.18) (end 108.595 95.14) (width 0.3) (layer "F.Cu") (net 5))
 (segment (start 112.02 94.84) (end 112.06 94.88) (width 0.3) (layer "F.Cu") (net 5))
 (segment (start 112.06 94.88) (end 108.805 94.88) (width 0.3) (layer "F.Cu") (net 5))
 (segment (start 110.57 63.27) (end 109.84 63.27) (width 0.75) (layer "F.Cu") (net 32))
 (segment (start 113.15 63.28) (end 110.58 63.28) (width 0.75) (layer "F.Cu") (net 32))
 (segment (start 110.58 63.28) (end 110.57 63.27) (width 0.75) (layer "F.Cu") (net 32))
 (segment (start 109.84 63.27) (end 101.81 71.3) (width 0.75) (layer "F.Cu") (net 32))
 (segment (start 109.43 71.3) (end 110.21 71.3) (width 0.75) (layer "B.Cu") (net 34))
 (segment (start 110.21 71.3) (end 113.15 68.36) (width 0.75) (layer "B.Cu") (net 34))
 (segment (start 94.19 71.3) (end 96.76 73.87) (width 0.75) (layer "B.Cu") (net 37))
 (segment (start 108.5 73.87) (end 113.15 78.52) (width 0.75) (layer "B.Cu") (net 37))
 (segment (start 96.76 73.87) (end 108.5 73.87) (width 0.75) (layer "B.Cu") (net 37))
 (segment (start 99.165 94.76) (end 99.235 94.83) (width 0.3) (layer "F.Cu") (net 8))
 (segment (start 96.325 94.785) (end 96.3 94.76) (width 0.3) (layer "F.Cu") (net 8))
 (segment (start 96.3 94.76) (end 99.165 94.76) (width 0.3) (layer "F.Cu") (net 8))
 (segment (start 106.89 71.3) (end 112.37 65.82) (width 0.75) (layer "B.Cu") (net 33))
 (segment (start 112.37 65.82) (end 113.15 65.82) (width 0.75) (layer "B.Cu") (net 33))
 (segment (start 104.34 56.85) (end 104.34 71.29) (width 0.75) (layer "B.Cu") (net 27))
 (segment (start 113.15 48.04) (end 104.34 56.85) (width 0.75) (layer "B.Cu") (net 27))
 (segment (start 104.34 71.29) (end 104.35 71.3) (width 0.75) (layer "B.Cu") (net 27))
 (segment (start 83.6 93.705) (end 79.49 93.705) (width 0.3) (layer "F.Cu") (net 1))
 (segment (start 79.49 93.705) (end 79.33 93.865) (width 0.3) (layer "F.Cu") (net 1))
 (segment (start 79.33 96.08) (end 80.38 97.13) (width 0.8) (layer "F.Cu") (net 1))
 (segment (start 80.38 97.13) (end 86.94 97.13) (width 0.8) (layer "F.Cu") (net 1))
 (segment (start 79.33 93.865) (end 79.33 96.08) (width 0.8) (layer "F.Cu") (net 1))
 (segment (start 104.76 80.6) (end 110.15 80.6) (width 0.75) (layer "B.Cu") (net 3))
 (segment (start 110.15 80.6) (end 113.15 83.6) (width 0.75) (layer "B.Cu") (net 3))
 (segment (start 85.21 90.84) (end 84.925 90.555) (width 0.3) (layer "F.Cu") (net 6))
 (segment (start 84.87 53.92) (end 84.87 57.86) (width 0.3) (layer "F.Cu") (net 6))
 (segment (start 83.68 90.555) (end 83.015 90.555) (width 0.3) (layer "F.Cu") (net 6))
 (segment (start 84.87 57.86) (end 87.75 60.74) (width 0.3) (layer "F.Cu") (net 6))
 (segment (start 84.465 93.065) (end 85.21 92.32) (width 0.3) (layer "F.Cu") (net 6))
 (segment (start 84.925 90.555) (end 83.68 90.555) (width 0.3) (layer "F.Cu") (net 6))
 (segment (start 79.25 64.01) (end 79.25 80.29) (width 0.8) (layer "F.Cu") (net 6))
 (segment (start 83.6 93.065) (end 84.465 93.065) (width 0.3) (layer "F.Cu") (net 6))
 (segment (start 82.52 60.74) (end 79.25 64.01) (width 0.8) (layer "F.Cu") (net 6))
 (segment (start 87.75 60.74) (end 82.52 60.74) (width 0.8) (layer "F.Cu") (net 6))
 (segment (start 85.21 92.32) (end 85.21 90.84) (width 0.3) (layer "F.Cu") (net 6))
 (segment (start 79.25 80.29) (end 79.25 86.79) (width 0.8) (layer "F.Cu") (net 6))
 (segment (start 83.015 90.555) (end 79.25 86.79) (width 0.3) (layer "F.Cu") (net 6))
 (segment (start 89.47 59.92) (end 89.47 90.48) (width 0.3) (layer "F.Cu") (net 14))
 (segment (start 93.11 94.12) (end 96.3 94.12) (width 0.3) (layer "F.Cu") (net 14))
 (segment (start 87.75 58.2) (end 89.47 59.92) (width 0.3) (layer "F.Cu") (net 14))
 (segment (start 89.47 90.48) (end 93.11 94.12) (width 0.3) (layer "F.Cu") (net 14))
 (segment (start 115.24 91.76) (end 115.24 93.06) (width 0.3) (layer "F.Cu") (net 4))
 (segment (start 115.25 91.75) (end 115.24 91.76) (width 0.3) (layer "F.Cu") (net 4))
 (segment (start 114.06 94.24) (end 112.06 94.24) (width 0.3) (layer "F.Cu") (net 4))
 (segment (start 113.15 70.9) (end 115.25 73) (width 0.3) (layer "F.Cu") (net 4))
 (segment (start 115.25 73) (end 115.25 91.75) (width 0.3) (layer "F.Cu") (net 4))
 (segment (start 115.24 93.06) (end 114.06 94.24) (width 0.3) (layer "F.Cu") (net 4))
 (segment (start 87.75 91.22) (end 87.75 92.86) (width 0.8) (layer "F.Cu") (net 25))
 (segment (start 87.75 92.86) (end 92.02 97.13) (width 0.8) (layer "F.Cu") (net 25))
 (segment (start 113.8 97.85) (end 116.3 95.35) (width 0.75) (layer "F.Cu") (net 7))
 (segment (start 113.15 60.74) (end 115.5 60.74) (width 0.75) (layer "F.Cu") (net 7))
 (segment (start 106.055 95.14) (end 106.055 96.585) (width 0.75) (layer "F.Cu") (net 7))
 (segment (start 105.985 95.07) (end 106.055 95.14) (width 0.75) (layer "F.Cu") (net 7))
 (segment (start 116.3 95.35) (end 116.3 93.7) (width 0.75) (layer "F.Cu") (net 7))
 (segment (start 101.775 94.83) (end 106.195 94.83) (width 0.8) (layer "F.Cu") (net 7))
 (segment (start 115.5 60.74) (end 116.3 61.54) (width 0.75) (layer "F.Cu") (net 7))
 (segment (start 106.195 94.83) (end 106.255 94.89) (width 0.8) (layer "F.Cu") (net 7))
 (segment (start 106.055 96.585) (end 107.32 97.85) (width 0.75) (layer "F.Cu") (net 7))
 (segment (start 116.3 61.54) (end 116.3 93.7) (width 0.75) (layer "F.Cu") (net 7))
 (segment (start 116.3 93.7) (end 116.27 93.7) (width 0.75) (layer "F.Cu") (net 7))
 (segment (start 107.32 97.85) (end 113.8 97.85) (width 0.75) (layer "F.Cu") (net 7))
 (segment (start 96.73 61.92) (end 113.15 45.5) (width 0.75) (layer "B.Cu") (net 26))
 (segment (start 96.73 71.3) (end 96.73 61.92) (width 0.75) (layer "B.Cu") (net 26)))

